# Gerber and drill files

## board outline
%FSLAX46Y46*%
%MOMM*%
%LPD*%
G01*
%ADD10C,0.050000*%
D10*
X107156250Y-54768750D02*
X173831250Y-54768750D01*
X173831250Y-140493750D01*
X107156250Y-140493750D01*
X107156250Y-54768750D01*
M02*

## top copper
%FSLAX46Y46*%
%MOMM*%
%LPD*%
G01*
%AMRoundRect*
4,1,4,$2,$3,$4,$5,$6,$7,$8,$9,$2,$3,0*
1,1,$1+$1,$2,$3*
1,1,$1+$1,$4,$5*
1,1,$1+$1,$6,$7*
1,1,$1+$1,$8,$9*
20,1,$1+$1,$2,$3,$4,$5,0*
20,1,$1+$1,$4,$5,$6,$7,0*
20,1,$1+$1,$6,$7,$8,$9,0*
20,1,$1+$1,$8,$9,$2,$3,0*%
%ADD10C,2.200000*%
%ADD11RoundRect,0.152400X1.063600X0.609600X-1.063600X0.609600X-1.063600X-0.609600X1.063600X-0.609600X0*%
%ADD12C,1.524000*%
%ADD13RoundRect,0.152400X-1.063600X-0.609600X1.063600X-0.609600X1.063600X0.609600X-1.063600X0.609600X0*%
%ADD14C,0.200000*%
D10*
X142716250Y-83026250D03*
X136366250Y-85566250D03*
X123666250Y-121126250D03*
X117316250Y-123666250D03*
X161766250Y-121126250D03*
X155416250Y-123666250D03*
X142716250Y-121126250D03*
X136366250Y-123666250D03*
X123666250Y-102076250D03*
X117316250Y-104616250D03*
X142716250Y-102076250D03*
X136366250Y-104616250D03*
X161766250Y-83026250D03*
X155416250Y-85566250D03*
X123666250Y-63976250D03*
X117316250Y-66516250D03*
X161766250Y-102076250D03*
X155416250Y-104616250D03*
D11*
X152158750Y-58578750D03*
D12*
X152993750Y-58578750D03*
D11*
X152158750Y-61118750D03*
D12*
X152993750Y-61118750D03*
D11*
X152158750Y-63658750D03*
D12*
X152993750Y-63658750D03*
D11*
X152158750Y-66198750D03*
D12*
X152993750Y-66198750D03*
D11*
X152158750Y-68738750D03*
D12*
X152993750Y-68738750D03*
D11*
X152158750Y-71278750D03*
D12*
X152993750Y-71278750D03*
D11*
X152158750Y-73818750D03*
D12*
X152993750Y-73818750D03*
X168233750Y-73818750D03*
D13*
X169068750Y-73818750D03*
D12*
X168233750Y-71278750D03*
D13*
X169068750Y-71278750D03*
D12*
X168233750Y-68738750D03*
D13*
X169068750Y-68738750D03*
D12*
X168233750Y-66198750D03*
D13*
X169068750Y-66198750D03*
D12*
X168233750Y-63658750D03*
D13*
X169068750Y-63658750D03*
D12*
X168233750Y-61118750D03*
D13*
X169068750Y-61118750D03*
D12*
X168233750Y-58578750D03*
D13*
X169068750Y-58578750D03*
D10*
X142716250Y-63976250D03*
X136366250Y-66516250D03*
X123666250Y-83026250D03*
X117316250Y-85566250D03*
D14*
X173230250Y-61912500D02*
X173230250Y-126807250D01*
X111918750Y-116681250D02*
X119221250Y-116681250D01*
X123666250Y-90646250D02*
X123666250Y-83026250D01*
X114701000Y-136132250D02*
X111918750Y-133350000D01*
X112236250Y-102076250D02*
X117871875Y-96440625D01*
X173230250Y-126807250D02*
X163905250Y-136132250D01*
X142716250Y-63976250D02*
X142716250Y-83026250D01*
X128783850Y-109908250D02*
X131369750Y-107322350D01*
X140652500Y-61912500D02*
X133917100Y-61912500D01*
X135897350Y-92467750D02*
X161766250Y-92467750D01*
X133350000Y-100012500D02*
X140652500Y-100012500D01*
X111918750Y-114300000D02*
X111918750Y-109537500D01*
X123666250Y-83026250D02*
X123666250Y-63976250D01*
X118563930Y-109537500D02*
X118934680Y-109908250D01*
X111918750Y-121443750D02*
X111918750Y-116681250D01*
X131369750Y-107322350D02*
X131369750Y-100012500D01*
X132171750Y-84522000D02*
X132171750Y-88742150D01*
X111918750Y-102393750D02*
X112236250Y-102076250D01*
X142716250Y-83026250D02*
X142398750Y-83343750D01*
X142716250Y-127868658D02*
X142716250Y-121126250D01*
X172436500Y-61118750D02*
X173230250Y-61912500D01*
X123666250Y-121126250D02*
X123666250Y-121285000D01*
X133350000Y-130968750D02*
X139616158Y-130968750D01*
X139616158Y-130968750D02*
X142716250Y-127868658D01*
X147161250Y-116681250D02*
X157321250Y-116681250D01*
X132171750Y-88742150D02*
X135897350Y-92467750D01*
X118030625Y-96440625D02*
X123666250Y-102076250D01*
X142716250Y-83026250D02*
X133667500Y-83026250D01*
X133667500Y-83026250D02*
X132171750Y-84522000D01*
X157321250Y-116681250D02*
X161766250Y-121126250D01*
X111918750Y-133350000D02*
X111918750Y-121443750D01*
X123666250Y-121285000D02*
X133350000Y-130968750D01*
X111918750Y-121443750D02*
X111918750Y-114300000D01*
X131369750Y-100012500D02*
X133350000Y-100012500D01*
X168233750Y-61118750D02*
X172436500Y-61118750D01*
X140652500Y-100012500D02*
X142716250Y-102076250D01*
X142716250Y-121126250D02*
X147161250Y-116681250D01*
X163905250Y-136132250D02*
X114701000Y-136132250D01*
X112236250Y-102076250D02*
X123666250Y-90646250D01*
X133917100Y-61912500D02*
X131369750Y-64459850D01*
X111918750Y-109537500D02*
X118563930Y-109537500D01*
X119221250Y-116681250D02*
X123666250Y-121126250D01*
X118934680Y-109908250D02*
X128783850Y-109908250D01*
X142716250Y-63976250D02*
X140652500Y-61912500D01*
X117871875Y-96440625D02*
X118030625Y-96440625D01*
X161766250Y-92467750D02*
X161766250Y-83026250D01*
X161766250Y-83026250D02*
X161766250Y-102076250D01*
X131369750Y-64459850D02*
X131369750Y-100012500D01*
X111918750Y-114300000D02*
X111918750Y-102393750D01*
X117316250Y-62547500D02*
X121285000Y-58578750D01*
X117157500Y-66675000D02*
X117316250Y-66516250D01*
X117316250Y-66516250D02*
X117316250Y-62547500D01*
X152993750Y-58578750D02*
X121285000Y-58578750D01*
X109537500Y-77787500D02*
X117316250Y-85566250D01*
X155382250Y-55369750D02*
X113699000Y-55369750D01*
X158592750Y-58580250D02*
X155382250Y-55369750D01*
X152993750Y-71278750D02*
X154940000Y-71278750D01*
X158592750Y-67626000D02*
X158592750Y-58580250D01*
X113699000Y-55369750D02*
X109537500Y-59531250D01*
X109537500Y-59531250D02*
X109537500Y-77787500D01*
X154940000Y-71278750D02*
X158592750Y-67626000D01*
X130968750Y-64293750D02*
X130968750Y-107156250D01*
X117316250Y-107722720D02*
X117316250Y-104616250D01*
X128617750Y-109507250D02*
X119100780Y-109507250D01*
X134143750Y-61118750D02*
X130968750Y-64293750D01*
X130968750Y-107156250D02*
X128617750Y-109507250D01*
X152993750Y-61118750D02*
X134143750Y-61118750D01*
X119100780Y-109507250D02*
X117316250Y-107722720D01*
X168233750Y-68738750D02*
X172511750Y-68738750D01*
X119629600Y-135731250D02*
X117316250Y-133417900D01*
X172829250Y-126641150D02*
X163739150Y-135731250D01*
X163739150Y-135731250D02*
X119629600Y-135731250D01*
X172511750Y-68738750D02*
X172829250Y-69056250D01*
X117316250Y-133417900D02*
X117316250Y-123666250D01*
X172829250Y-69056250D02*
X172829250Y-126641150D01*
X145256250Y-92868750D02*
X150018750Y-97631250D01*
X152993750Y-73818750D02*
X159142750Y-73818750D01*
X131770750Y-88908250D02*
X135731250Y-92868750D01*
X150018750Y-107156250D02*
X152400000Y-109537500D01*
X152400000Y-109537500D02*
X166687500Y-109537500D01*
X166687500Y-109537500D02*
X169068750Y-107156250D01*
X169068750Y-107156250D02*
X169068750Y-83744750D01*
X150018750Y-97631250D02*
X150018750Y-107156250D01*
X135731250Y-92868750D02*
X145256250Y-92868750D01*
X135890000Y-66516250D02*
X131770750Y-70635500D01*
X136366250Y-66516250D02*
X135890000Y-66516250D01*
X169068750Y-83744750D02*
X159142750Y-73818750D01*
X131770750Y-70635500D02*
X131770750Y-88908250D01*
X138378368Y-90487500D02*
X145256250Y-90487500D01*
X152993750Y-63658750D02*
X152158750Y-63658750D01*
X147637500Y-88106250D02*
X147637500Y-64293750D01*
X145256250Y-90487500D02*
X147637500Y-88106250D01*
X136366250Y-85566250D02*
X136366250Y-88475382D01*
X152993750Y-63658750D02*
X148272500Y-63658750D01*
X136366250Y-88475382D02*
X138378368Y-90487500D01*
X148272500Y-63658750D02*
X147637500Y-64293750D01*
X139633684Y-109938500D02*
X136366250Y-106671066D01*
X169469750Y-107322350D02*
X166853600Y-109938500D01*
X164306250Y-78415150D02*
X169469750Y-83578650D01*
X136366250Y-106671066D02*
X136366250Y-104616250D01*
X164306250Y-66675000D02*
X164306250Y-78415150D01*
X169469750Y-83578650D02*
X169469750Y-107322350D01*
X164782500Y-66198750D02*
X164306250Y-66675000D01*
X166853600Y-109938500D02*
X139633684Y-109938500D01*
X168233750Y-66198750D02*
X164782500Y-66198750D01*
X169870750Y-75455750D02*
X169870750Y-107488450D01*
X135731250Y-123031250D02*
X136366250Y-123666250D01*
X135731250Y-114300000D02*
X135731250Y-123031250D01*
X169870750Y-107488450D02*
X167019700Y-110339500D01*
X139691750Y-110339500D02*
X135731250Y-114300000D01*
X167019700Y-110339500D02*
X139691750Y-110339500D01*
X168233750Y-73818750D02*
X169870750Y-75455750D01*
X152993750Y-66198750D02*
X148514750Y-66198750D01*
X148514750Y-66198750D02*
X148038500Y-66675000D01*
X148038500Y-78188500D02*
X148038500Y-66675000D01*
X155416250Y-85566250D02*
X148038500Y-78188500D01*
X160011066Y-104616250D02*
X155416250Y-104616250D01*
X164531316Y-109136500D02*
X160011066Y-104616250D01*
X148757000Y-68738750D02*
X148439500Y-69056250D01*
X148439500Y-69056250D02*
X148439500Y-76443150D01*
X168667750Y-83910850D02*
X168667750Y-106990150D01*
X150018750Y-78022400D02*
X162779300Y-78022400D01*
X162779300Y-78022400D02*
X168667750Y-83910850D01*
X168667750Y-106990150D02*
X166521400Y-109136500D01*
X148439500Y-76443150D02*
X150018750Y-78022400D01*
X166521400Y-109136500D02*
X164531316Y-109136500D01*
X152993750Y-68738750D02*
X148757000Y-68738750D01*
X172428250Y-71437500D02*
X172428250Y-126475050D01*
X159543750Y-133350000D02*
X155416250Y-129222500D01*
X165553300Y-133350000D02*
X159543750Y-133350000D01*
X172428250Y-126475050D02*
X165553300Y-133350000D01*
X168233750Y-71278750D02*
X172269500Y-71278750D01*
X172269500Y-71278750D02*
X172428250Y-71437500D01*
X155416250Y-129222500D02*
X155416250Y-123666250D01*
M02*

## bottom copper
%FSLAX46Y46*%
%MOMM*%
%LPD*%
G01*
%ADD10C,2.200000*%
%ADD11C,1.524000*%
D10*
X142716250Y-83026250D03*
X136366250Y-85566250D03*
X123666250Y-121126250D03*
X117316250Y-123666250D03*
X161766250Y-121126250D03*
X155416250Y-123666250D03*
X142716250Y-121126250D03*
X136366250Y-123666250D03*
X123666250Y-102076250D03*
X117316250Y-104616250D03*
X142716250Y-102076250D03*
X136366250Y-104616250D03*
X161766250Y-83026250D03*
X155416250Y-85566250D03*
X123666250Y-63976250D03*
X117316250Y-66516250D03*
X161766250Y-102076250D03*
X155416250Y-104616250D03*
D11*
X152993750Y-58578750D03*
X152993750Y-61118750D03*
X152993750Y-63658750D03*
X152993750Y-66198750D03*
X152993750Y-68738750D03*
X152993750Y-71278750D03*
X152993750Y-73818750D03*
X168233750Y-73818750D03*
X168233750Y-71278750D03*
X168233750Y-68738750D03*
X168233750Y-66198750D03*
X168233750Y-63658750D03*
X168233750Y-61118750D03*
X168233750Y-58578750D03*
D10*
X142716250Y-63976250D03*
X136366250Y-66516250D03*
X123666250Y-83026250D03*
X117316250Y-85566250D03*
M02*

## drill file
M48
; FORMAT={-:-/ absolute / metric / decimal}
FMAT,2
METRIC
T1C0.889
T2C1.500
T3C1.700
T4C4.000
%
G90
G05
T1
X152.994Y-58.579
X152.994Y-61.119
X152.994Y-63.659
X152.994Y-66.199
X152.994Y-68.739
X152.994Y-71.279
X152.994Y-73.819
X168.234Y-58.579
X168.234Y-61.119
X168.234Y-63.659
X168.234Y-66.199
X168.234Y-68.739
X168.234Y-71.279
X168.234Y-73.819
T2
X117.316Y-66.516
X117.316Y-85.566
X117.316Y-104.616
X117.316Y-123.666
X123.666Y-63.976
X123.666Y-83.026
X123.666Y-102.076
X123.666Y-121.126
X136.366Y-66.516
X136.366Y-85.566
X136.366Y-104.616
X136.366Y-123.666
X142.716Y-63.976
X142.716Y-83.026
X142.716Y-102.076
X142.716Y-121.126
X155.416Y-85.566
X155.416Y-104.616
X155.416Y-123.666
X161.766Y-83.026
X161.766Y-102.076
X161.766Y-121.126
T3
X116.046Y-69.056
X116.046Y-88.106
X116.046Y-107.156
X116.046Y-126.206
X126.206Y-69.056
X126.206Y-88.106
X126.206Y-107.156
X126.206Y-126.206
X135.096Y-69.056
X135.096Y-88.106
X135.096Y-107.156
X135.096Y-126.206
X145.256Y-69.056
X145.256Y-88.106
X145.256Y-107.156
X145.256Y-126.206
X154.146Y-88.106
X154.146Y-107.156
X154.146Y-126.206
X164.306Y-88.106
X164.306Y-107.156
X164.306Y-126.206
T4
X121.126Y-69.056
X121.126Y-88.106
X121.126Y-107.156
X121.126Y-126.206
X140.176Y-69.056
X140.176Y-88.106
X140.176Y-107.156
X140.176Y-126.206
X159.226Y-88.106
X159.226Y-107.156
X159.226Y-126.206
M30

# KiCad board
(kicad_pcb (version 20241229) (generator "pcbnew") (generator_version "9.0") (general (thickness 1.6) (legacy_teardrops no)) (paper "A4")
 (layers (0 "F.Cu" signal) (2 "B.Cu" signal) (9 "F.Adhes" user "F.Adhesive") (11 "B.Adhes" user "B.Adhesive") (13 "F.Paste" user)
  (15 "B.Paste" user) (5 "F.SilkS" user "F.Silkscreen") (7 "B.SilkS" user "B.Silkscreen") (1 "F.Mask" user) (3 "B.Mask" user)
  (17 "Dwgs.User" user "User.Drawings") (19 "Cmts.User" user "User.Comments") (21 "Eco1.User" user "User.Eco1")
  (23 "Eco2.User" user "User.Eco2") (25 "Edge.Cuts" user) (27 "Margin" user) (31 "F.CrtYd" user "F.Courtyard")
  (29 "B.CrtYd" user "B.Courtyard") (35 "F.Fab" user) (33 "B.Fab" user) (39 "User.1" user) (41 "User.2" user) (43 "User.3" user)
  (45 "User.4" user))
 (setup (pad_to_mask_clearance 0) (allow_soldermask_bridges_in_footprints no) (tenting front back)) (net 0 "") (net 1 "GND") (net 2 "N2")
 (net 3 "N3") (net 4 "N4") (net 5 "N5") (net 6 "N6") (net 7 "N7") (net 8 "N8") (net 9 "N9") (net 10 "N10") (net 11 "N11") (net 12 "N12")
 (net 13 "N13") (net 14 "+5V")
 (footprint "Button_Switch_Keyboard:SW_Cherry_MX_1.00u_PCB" (layer "F.Cu") (at 142.71625 83.02625)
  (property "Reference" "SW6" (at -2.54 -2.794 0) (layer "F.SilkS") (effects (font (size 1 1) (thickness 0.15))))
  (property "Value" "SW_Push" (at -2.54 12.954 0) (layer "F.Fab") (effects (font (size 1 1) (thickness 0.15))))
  (pad "" np_thru_hole circle (at -7.62 5.08) (size 1.7 1.7) (drill 1.7) (layers "*.Cu" "*.Mask"))
  (pad "" np_thru_hole circle (at -2.54 5.08) (size 4 4) (drill 4) (layers "*.Cu" "*.Mask"))
  (pad "" np_thru_hole circle (at 2.54 5.08) (size 1.7 1.7) (drill 1.7) (layers "*.Cu" "*.Mask"))
  (pad "1" thru_hole circle (at 0 0) (size 2.2 2.2) (drill 1.5) (layers "*.Cu" "*.Mask") (remove_unused_layers no) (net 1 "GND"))
  (pad "2" thru_hole circle (at -6.35 2.54) (size 2.2 2.2) (drill 1.5) (layers "*.Cu" "*.Mask") (remove_unused_layers no) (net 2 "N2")))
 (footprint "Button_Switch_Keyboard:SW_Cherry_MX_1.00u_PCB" (layer "F.Cu") (at 123.66625 121.12625)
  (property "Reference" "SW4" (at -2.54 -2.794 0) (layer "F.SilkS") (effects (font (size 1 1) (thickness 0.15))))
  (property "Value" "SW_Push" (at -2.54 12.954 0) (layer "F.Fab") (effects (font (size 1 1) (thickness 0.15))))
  (pad "" np_thru_hole circle (at -7.62 5.08) (size 1.7 1.7) (drill 1.7) (layers "*.Cu" "*.Mask"))
  (pad "" np_thru_hole circle (at -2.54 5.08) (size 4 4) (drill 4) (layers "*.Cu" "*.Mask"))
  (pad "" np_thru_hole circle (at 2.54 5.08) (size 1.7 1.7) (drill 1.7) (layers "*.Cu" "*.Mask"))
  (pad "1" thru_hole circle (at 0 0) (size 2.2 2.2) (drill 1.5) (layers "*.Cu" "*.Mask") (remove_unused_layers no) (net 1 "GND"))
  (pad "2" thru_hole circle (at -6.35 2.54) (size 2.2 2.2) (drill 1.5) (layers "*.Cu" "*.Mask") (remove_unused_layers no) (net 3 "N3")))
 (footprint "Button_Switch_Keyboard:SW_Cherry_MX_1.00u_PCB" (layer "F.Cu") (at 161.76625 121.12625)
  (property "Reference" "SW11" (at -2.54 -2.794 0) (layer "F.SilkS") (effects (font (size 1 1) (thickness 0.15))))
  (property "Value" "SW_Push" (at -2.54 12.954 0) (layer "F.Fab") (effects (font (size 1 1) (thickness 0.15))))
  (pad "" np_thru_hole circle (at -7.62 5.08) (size 1.7 1.7) (drill 1.7) (layers "*.Cu" "*.Mask"))
  (pad "" np_thru_hole circle (at -2.54 5.08) (size 4 4) (drill 4) (layers "*.Cu" "*.Mask"))
  (pad "" np_thru_hole circle (at 2.54 5.08) (size 1.7 1.7) (drill 1.7) (layers "*.Cu" "*.Mask"))
  (pad "1" thru_hole circle (at 0 0) (size 2.2 2.2) (drill 1.5) (layers "*.Cu" "*.Mask") (remove_unused_layers no) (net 1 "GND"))
  (pad "2" thru_hole circle (at -6.35 2.54) (size 2.2 2.2) (drill 1.5) (layers "*.Cu" "*.Mask") (remove_unused_layers no) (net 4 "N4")))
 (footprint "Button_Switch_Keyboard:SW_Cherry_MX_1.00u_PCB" (layer "F.Cu") (at 142.71625 121.12625)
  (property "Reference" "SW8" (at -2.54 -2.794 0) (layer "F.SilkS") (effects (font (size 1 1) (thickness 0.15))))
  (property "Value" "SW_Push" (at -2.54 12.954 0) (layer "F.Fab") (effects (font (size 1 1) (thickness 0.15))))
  (pad "" np_thru_hole circle (at -7.62 5.08) (size 1.7 1.7) (drill 1.7) (layers "*.Cu" "*.Mask"))
  (pad "" np_thru_hole circle (at -2.54 5.08) (size 4 4) (drill 4) (layers "*.Cu" "*.Mask"))
  (pad "" np_thru_hole circle (at 2.54 5.08) (size 1.7 1.7) (drill 1.7) (layers "*.Cu" "*.Mask"))
  (pad "1" thru_hole circle (at 0 0) (size 2.2 2.2) (drill 1.5) (layers "*.Cu" "*.Mask") (remove_unused_layers no) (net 1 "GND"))
  (pad "2" thru_hole circle (at -6.35 2.54) (size 2.2 2.2) (drill 1.5) (layers "*.Cu" "*.Mask") (remove_unused_layers no) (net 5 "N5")))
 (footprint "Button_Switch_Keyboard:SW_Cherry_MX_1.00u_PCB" (layer "F.Cu") (at 123.66625 102.07625)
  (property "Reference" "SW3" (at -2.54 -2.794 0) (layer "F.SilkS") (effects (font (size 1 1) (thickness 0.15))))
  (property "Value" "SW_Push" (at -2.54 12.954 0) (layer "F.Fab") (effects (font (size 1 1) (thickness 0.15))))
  (pad "" np_thru_hole circle (at -7.62 5.08) (size 1.7 1.7) (drill 1.7) (layers "*.Cu" "*.Mask"))
  (pad "" np_thru_hole circle (at -2.54 5.08) (size 4 4) (drill 4) (layers "*.Cu" "*.Mask"))
  (pad "" np_thru_hole circle (at 2.54 5.08) (size 1.7 1.7) (drill 1.7) (layers "*.Cu" "*.Mask"))
  (pad "1" thru_hole circle (at 0 0) (size 2.2 2.2) (drill 1.5) (layers "*.Cu" "*.Mask") (remove_unused_layers no) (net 1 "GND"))
  (pad "2" thru_hole circle (at -6.35 2.54) (size 2.2 2.2) (drill 1.5) (layers "*.Cu" "*.Mask") (remove_unused_layers no) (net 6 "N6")))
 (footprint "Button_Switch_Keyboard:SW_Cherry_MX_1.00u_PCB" (layer "F.Cu") (at 142.71625 102.07625)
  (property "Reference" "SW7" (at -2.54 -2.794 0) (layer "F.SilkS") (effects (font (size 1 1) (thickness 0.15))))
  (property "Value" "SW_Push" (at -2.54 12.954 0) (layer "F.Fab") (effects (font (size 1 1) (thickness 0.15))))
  (pad "" np_thru_hole circle (at -7.62 5.08) (size 1.7 1.7) (drill 1.7) (layers "*.Cu" "*.Mask"))
  (pad "" np_thru_hole circle (at -2.54 5.08) (size 4 4) (drill 4) (layers "*.Cu" "*.Mask"))
  (pad "" np_thru_hole circle (at 2.54 5.08) (size 1.7 1.7) (drill 1.7) (layers "*.Cu" "*.Mask"))
  (pad "1" thru_hole circle (at 0 0) (size 2.2 2.2) (drill 1.5) (layers "*.Cu" "*.Mask") (remove_unused_layers no) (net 1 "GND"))
  (pad "2" thru_hole circle (at -6.35 2.54) (size 2.2 2.2) (drill 1.5) (layers "*.Cu" "*.Mask") (remove_unused_layers no) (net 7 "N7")))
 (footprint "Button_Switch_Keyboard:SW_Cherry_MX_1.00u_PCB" (layer "F.Cu") (at 161.76625 83.02625)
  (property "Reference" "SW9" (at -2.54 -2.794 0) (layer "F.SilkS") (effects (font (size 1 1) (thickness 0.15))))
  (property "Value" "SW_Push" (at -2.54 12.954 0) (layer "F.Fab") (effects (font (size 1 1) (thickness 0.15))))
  (pad "" np_thru_hole circle (at -7.62 5.08) (size 1.7 1.7) (drill 1.7) (layers "*.Cu" "*.Mask"))
  (pad "" np_thru_hole circle (at -2.54 5.08) (size 4 4) (drill 4) (layers "*.Cu" "*.Mask"))
  (pad "" np_thru_hole circle (at 2.54 5.08) (size 1.7 1.7) (drill 1.7) (layers "*.Cu" "*.Mask"))
  (pad "1" thru_hole circle (at 0 0) (size 2.2 2.2) (drill 1.5) (layers "*.Cu" "*.Mask") (remove_unused_layers no) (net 1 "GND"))
  (pad "2" thru_hole circle (at -6.35 2.54) (size 2.2 2.2) (drill 1.5) (layers "*.Cu" "*.Mask") (remove_unused_layers no) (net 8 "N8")))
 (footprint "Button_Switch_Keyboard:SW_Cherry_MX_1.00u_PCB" (layer "F.Cu") (at 123.66625 63.97625)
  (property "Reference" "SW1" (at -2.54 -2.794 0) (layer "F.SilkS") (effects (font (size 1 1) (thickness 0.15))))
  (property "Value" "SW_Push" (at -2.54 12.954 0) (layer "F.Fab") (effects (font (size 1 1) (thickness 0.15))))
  (pad "" np_thru_hole circle (at -7.62 5.08) (size 1.7 1.7) (drill 1.7) (layers "*.Cu" "*.Mask"))
  (pad "" np_thru_hole circle (at -2.54 5.08) (size 4 4) (drill 4) (layers "*.Cu" "*.Mask"))
  (pad "" np_thru_hole circle (at 2.54 5.08) (size 1.7 1.7) (drill 1.7) (layers "*.Cu" "*.Mask"))
  (pad "1" thru_hole circle (at 0 0) (size 2.2 2.2) (drill 1.5) (layers "*.Cu" "*.Mask") (remove_unused_layers no) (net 1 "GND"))
  (pad "2" thru_hole circle (at -6.35 2.54) (size 2.2 2.2) (drill 1.5) (layers "*.Cu" "*.Mask") (remove_unused_layers no) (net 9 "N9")))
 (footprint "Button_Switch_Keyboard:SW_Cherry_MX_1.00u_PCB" (layer "F.Cu") (at 161.76625 102.07625)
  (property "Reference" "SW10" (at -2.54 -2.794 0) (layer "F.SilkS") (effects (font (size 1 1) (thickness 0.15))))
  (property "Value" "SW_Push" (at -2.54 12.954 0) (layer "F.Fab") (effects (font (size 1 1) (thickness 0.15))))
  (pad "" np_thru_hole circle (at -7.62 5.08) (size 1.7 1.7) (drill 1.7) (layers "*.Cu" "*.Mask"))
  (pad "" np_thru_hole circle (at -2.54 5.08) (size 4 4) (drill 4) (layers "*.Cu" "*.Mask"))
  (pad "" np_thru_hole circle (at 2.54 5.08) (size 1.7 1.7) (drill 1.7) (layers "*.Cu" "*.Mask"))
  (pad "1" thru_hole circle (at 0 0) (size 2.2 2.2) (drill 1.5) (layers "*.Cu" "*.Mask") (remove_unused_layers no) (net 1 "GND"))
  (pad "2" thru_hole circle (at -6.35 2.54) (size 2.2 2.2) (drill 1.5) (layers "*.Cu" "*.Mask") (remove_unused_layers no) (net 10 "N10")))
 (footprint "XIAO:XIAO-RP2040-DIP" (layer "F.Cu") (at 160.61375 66.19875)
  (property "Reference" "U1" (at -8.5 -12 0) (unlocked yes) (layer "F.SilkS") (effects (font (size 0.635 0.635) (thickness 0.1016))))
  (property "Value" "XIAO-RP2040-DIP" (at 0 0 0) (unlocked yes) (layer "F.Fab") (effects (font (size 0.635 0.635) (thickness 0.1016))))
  (pad "1" smd roundrect (at -8.455 -7.62 180) (size 2.432 1.524) (layers "F.Cu" "F.Mask") (roundrect_rratio 0.1) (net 9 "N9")
   (thermal_bridge_angle 45))
  (pad "1" thru_hole circle (at -7.62 -7.62 180) (size 1.524 1.524) (drill 0.889) (layers "*.Cu" "*.Mask") (remove_unused_layers no)
   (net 9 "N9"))
  (pad "2" smd roundrect (at -8.455 -5.08 180) (size 2.432 1.524) (layers "F.Cu" "F.Mask") (roundrect_rratio 0.1) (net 6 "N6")
   (thermal_bridge_angle 45))
  (pad "2" thru_hole circle (at -7.62 -5.08 180) (size 1.524 1.524) (drill 0.889) (layers "*.Cu" "*.Mask") (remove_unused_layers no)
   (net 6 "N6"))
  (pad "3" smd roundrect (at -8.455 -2.54 180) (size 2.432 1.524) (layers "F.Cu" "F.Mask") (roundrect_rratio 0.1) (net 2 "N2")
   (thermal_bridge_angle 45))
  (pad "3" thru_hole circle (at -7.62 -2.54 180) (size 1.524 1.524) (drill 0.889) (layers "*.Cu" "*.Mask") (remove_unused_layers no)
   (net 2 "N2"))
  (pad "4" smd roundrect (at -8.455 0 180) (size 2.432 1.524) (layers "F.Cu" "F.Mask") (roundrect_rratio 0.1) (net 8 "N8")
   (thermal_bridge_angle 45))
  (pad "4" thru_hole circle (at -7.62 0 180) (size 1.524 1.524) (drill 0.889) (layers "*.Cu" "*.Mask") (remove_unused_layers no)
   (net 8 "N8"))
  (pad "5" smd roundrect (at -8.455 2.54 180) (size 2.432 1.524) (layers "F.Cu" "F.Mask") (roundrect_rratio 0.1) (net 10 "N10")
   (thermal_bridge_angle 45))
  (pad "5" thru_hole circle (at -7.62 2.54 180) (size 1.524 1.524) (drill 0.889) (layers "*.Cu" "*.Mask") (remove_unused_layers no)
   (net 10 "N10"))
  (pad "6" smd roundrect (at -8.455 5.08 180) (size 2.432 1.524) (layers "F.Cu" "F.Mask") (roundrect_rratio 0.1) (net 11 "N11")
   (thermal_bridge_angle 45))
  (pad "6" thru_hole circle (at -7.62 5.08 180) (size 1.524 1.524) (drill 0.889) (layers "*.Cu" "*.Mask") (remove_unused_layers no)
   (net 11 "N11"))
  (pad "7" smd roundrect (at -8.455 7.62 180) (size 2.432 1.524) (layers "F.Cu" "F.Mask") (roundrect_rratio 0.1) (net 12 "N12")
   (thermal_bridge_angle 45))
  (pad "7" thru_hole circle (at -7.62 7.62 180) (size 1.524 1.524) (drill 0.889) (layers "*.Cu" "*.Mask") (remove_unused_layers no)
   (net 12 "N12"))
  (pad "8" thru_hole circle (at 7.62 7.62) (size 1.524 1.524) (drill 0.889) (layers "*.Cu" "*.Mask") (remove_unused_layers no) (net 5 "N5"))
  (pad "8" smd roundrect (at 8.455 7.62) (size 2.432 1.524) (layers "F.Cu" "F.Mask") (roundrect_rratio 0.1) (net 5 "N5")
   (thermal_bridge_angle 45))
  (pad "9" thru_hole circle (at 7.62 5.08) (size 1.524 1.524) (drill 0.889) (layers "*.Cu" "*.Mask") (remove_unused_layers no) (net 4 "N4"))
  (pad "9" smd roundrect (at 8.455 5.08) (size 2.432 1.524) (layers "F.Cu" "F.Mask") (roundrect_rratio 0.1) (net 4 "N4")
   (thermal_bridge_angle 45))
  (pad "10" thru_hole circle (at 7.62 2.54) (size 1.524 1.524) (drill 0.889) (layers "*.Cu" "*.Mask") (remove_unused_layers no) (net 3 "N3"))
  (pad "10" smd roundrect (at 8.455 2.54) (size 2.432 1.524) (layers "F.Cu" "F.Mask") (roundrect_rratio 0.1) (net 3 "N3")
   (thermal_bridge_angle 45))
  (pad "11" thru_hole circle (at 7.62 0) (size 1.524 1.524) (drill 0.889) (layers "*.Cu" "*.Mask") (remove_unused_layers no) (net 7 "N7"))
  (pad "11" smd roundrect (at 8.455 0) (size 2.432 1.524) (layers "F.Cu" "F.Mask") (roundrect_rratio 0.1) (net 7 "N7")
   (thermal_bridge_angle 45))
  (pad "12" thru_hole circle (at 7.62 -2.54) (size 1.524 1.524) (drill 0.889) (layers "*.Cu" "*.Mask") (remove_unused_layers no)
   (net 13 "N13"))
  (pad "12" smd roundrect (at 8.455 -2.54) (size 2.432 1.524) (layers "F.Cu" "F.Mask") (roundrect_rratio 0.1) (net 13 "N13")
   (thermal_bridge_angle 45))
  (pad "13" thru_hole circle (at 7.62 -5.08) (size 1.524 1.524) (drill 0.889) (layers "*.Cu" "*.Mask") (remove_unused_layers no)
   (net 1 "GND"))
  (pad "13" smd roundrect (at 8.455 -5.08) (size 2.432 1.524) (layers "F.Cu" "F.Mask") (roundrect_rratio 0.1) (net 1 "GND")
   (thermal_bridge_angle 45))
  (pad "14" thru_hole circle (at 7.62 -7.62) (size 1.524 1.524) (drill 0.889) (layers "*.Cu" "*.Mask") (remove_unused_layers no)
   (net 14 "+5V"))
  (pad "14" smd roundrect (at 8.455 -7.62) (size 2.432 1.524) (layers "F.Cu" "F.Mask") (roundrect_rratio 0.1) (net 14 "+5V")
   (thermal_bridge_angle 45)))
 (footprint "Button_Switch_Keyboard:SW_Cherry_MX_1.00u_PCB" (layer "F.Cu") (at 142.71625 63.97625)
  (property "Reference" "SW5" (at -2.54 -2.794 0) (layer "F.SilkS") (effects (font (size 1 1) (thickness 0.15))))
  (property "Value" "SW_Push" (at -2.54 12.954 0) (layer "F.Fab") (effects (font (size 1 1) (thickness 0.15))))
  (pad "" np_thru_hole circle (at -7.62 5.08) (size 1.7 1.7) (drill 1.7) (layers "*.Cu" "*.Mask"))
  (pad "" np_thru_hole circle (at -2.54 5.08) (size 4 4) (drill 4) (layers "*.Cu" "*.Mask"))
  (pad "" np_thru_hole circle (at 2.54 5.08) (size 1.7 1.7) (drill 1.7) (layers "*.Cu" "*.Mask"))
  (pad "1" thru_hole circle (at 0 0) (size 2.2 2.2) (drill 1.5) (layers "*.Cu" "*.Mask") (remove_unused_layers no) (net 1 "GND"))
  (pad "2" thru_hole circle (at -6.35 2.54) (size 2.2 2.2) (drill 1.5) (layers "*.Cu" "*.Mask") (remove_unused_layers no) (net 12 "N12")))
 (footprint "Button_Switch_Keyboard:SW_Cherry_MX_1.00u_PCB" (layer "F.Cu") (at 123.66625 83.02625)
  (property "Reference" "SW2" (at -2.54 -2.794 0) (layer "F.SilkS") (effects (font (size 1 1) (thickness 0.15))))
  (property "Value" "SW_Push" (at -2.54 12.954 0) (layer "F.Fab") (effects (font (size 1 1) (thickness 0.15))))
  (pad "" np_thru_hole circle (at -7.62 5.08) (size 1.7 1.7) (drill 1.7) (layers "*.Cu" "*.Mask"))
  (pad "" np_thru_hole circle (at -2.54 5.08) (size 4 4) (drill 4) (layers "*.Cu" "*.Mask"))
  (pad "" np_thru_hole circle (at 2.54 5.08) (size 1.7 1.7) (drill 1.7) (layers "*.Cu" "*.Mask"))
  (pad "1" thru_hole circle (at 0 0) (size 2.2 2.2) (drill 1.5) (layers "*.Cu" "*.Mask") (remove_unused_layers no) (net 1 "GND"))
  (pad "2" thru_hole circle (at -6.35 2.54) (size 2.2 2.2) (drill 1.5) (layers "*.Cu" "*.Mask") (remove_unused_layers no) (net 11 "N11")))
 (gr_rect (start 107.15625 54.76875) (end 173.83125 140.49375) (stroke (width 0.05) (type default)) (fill no) (layer "Edge.Cuts"))
 (segment (start 173.23025 61.9125) (end 173.23025 126.80725) (width 0.2) (layer "F.Cu") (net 1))
 (segment (start 111.91875 116.68125) (end 119.22125 116.68125) (width 0.2) (layer "F.Cu") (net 1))
 (segment (start 123.66625 90.64625) (end 123.66625 83.02625) (width 0.2) (layer "F.Cu") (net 1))
 (segment (start 114.701 136.13225) (end 111.91875 133.35) (width 0.2) (layer "F.Cu") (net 1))
 (segment (start 112.23625 102.07625) (end 117.871875 96.440625) (width 0.2) (layer "F.Cu") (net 1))
 (segment (start 173.23025 126.80725) (end 163.90525 136.13225) (width 0.2) (layer "F.Cu") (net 1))
 (segment (start 142.71625 63.97625) (end 142.71625 83.02625) (width 0.2) (layer "F.Cu") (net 1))
 (segment (start 128.78385 109.90825) (end 131.36975 107.32235) (width 0.2) (layer "F.Cu") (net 1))
 (segment (start 140.6525 61.9125) (end 133.9171 61.9125) (width 0.2) (layer "F.Cu") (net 1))
 (segment (start 135.89735 92.46775) (end 161.76625 92.46775) (width 0.2) (layer "F.Cu") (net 1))
 (segment (start 133.35 100.0125) (end 140.6525 100.0125) (width 0.2) (layer "F.Cu") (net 1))
 (segment (start 111.91875 114.3) (end 111.91875 109.5375) (width 0.2) (layer "F.Cu") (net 1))
 (segment (start 123.66625 83.02625) (end 123.66625 63.97625) (width 0.2) (layer "F.Cu") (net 1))
 (segment (start 118.56393 109.5375) (end 118.93468 109.90825) (width 0.2) (layer "F.Cu") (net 1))
 (segment (start 111.91875 121.44375) (end 111.91875 116.68125) (width 0.2) (layer "F.Cu") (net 1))
 (segment (start 131.36975 107.32235) (end 131.36975 100.0125) (width 0.2) (layer "F.Cu") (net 1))
 (segment (start 132.17175 84.522) (end 132.17175 88.74215) (width 0.2) (layer "F.Cu") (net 1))
 (segment (start 111.91875 102.39375) (end 112.23625 102.07625) (width 0.2) (layer "F.Cu") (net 1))
 (segment (start 142.71625 83.02625) (end 142.39875 83.34375) (width 0.2) (layer "F.Cu") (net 1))
 (segment (start 142.71625 127.868658) (end 142.71625 121.12625) (width 0.2) (layer "F.Cu") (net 1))
 (segment (start 172.4365 61.11875) (end 173.23025 61.9125) (width 0.2) (layer "F.Cu") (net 1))
 (segment (start 123.66625 121.12625) (end 123.66625 121.285) (width 0.2) (layer "F.Cu") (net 1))
 (segment (start 133.35 130.96875) (end 139.616158 130.96875) (width 0.2) (layer "F.Cu") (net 1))
 (segment (start 139.616158 130.96875) (end 142.71625 127.868658) (width 0.2) (layer "F.Cu") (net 1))
 (segment (start 147.16125 116.68125) (end 157.32125 116.68125) (width 0.2) (layer "F.Cu") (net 1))
 (segment (start 132.17175 88.74215) (end 135.89735 92.46775) (width 0.2) (layer "F.Cu") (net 1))
 (segment (start 118.030625 96.440625) (end 123.66625 102.07625) (width 0.2) (layer "F.Cu") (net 1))
 (segment (start 142.71625 83.02625) (end 133.6675 83.02625) (width 0.2) (layer "F.Cu") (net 1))
 (segment (start 133.6675 83.02625) (end 132.17175 84.522) (width 0.2) (layer "F.Cu") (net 1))
 (segment (start 157.32125 116.68125) (end 161.76625 121.12625) (width 0.2) (layer "F.Cu") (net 1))
 (segment (start 111.91875 133.35) (end 111.91875 121.44375) (width 0.2) (layer "F.Cu") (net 1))
 (segment (start 123.66625 121.285) (end 133.35 130.96875) (width 0.2) (layer "F.Cu") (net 1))
 (segment (start 111.91875 121.44375) (end 111.91875 114.3) (width 0.2) (layer "F.Cu") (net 1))
 (segment (start 131.36975 100.0125) (end 133.35 100.0125) (width 0.2) (layer "F.Cu") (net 1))
 (segment (start 168.23375 61.11875) (end 172.4365 61.11875) (width 0.2) (layer "F.Cu") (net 1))
 (segment (start 140.6525 100.0125) (end 142.71625 102.07625) (width 0.2) (layer "F.Cu") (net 1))
 (segment (start 142.71625 121.12625) (end 147.16125 116.68125) (width 0.2) (layer "F.Cu") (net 1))
 (segment (start 163.90525 136.13225) (end 114.701 136.13225) (width 0.2) (layer "F.Cu") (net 1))
 (segment (start 112.23625 102.07625) (end 123.66625 90.64625) (width 0.2) (layer "F.Cu") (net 1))
 (segment (start 133.9171 61.9125) (end 131.36975 64.45985) (width 0.2) (layer "F.Cu") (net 1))
 (segment (start 111.91875 109.5375) (end 118.56393 109.5375) (width 0.2) (layer "F.Cu") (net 1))
 (segment (start 119.22125 116.68125) (end 123.66625 121.12625) (width 0.2) (layer "F.Cu") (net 1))
 (segment (start 118.93468 109.90825) (end 128.78385 109.90825) (width 0.2) (layer "F.Cu") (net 1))
 (segment (start 142.71625 63.97625) (end 140.6525 61.9125) (width 0.2) (layer "F.Cu") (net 1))
 (segment (start 117.871875 96.440625) (end 118.030625 96.440625) (width 0.2) (layer "F.Cu") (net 1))
 (segment (start 161.76625 92.46775) (end 161.76625 83.02625) (width 0.2) (layer "F.Cu") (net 1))
 (segment (start 161.76625 83.02625) (end 161.76625 102.07625) (width 0.2) (layer "F.Cu") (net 1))
 (segment (start 131.36975 64.45985) (end 131.36975 100.0125) (width 0.2) (layer "F.Cu") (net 1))
 (segment (start 111.91875 114.3) (end 111.91875 102.39375) (width 0.2) (layer "F.Cu") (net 1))
 (segment (start 117.31625 62.5475) (end 121.285 58.57875) (width 0.2) (layer "F.Cu") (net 9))
 (segment (start 117.1575 66.675) (end 117.31625 66.51625) (width 0.2) (layer "F.Cu") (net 9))
 (segment (start 117.31625 66.51625) (end 117.31625 62.5475) (width 0.2) (layer "F.Cu") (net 9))
 (segment (start 152.99375 58.57875) (end 121.285 58.57875) (width 0.2) (layer "F.Cu") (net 9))
 (segment (start 109.5375 77.7875) (end 117.31625 85.56625) (width 0.2) (layer "F.Cu") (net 11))
 (segment (start 155.38225 55.36975) (end 113.699 55.36975) (width 0.2) (layer "F.Cu") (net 11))
 (segment (start 158.59275 58.58025) (end 155.38225 55.36975) (width 0.2) (layer "F.Cu") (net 11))
 (segment (start 152.99375 71.27875) (end 154.94 71.27875) (width 0.2) (layer "F.Cu") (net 11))
 (segment (start 158.59275 67.626) (end 158.59275 58.58025) (width 0.2) (layer "F.Cu") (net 11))
 (segment (start 113.699 55.36975) (end 109.5375 59.53125) (width 0.2) (layer "F.Cu") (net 11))
 (segment (start 109.5375 59.53125) (end 109.5375 77.7875) (width 0.2) (layer "F.Cu") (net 11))
 (segment (start 154.94 71.27875) (end 158.59275 67.626) (width 0.2) (layer "F.Cu") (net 11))
 (segment (start 130.96875 64.29375) (end 130.96875 107.15625) (width 0.2) (layer "F.Cu") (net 6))
 (segment (start 117.31625 107.72272) (end 117.31625 104.61625) (width 0.2) (layer "F.Cu") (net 6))
 (segment (start 128.61775 109.50725) (end 119.10078 109.50725) (width 0.2) (layer "F.Cu") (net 6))
 (segment (start 134.14375 61.11875) (end 130.96875 64.29375) (width 0.2) (layer "F.Cu") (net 6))
 (segment (start 130.96875 107.15625) (end 128.61775 109.50725) (width 0.2) (layer "F.Cu") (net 6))
 (segment (start 152.99375 61.11875) (end 134.14375 61.11875) (width 0.2) (layer "F.Cu") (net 6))
 (segment (start 119.10078 109.50725) (end 117.31625 107.72272) (width 0.2) (layer "F.Cu") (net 6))
 (segment (start 168.23375 68.73875) (end 172.51175 68.73875) (width 0.2) (layer "F.Cu") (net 3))
 (segment (start 119.6296 135.73125) (end 117.31625 133.4179) (width 0.2) (layer "F.Cu") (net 3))
 (segment (start 172.82925 126.64115) (end 163.73915 135.73125) (width 0.2) (layer "F.Cu") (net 3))
 (segment (start 163.73915 135.73125) (end 119.6296 135.73125) (width 0.2) (layer "F.Cu") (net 3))
 (segment (start 172.51175 68.73875) (end 172.82925 69.05625) (width 0.2) (layer "F.Cu") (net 3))
 (segment (start 117.31625 133.4179) (end 117.31625 123.66625) (width 0.2) (layer "F.Cu") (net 3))
 (segment (start 172.82925 69.05625) (end 172.82925 126.64115) (width 0.2) (layer "F.Cu") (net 3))
 (segment (start 145.25625 92.86875) (end 150.01875 97.63125) (width 0.2) (layer "F.Cu") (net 12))
 (segment (start 152.99375 73.81875) (end 159.14275 73.81875) (width 0.2) (layer "F.Cu") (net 12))
 (segment (start 131.77075 88.90825) (end 135.73125 92.86875) (width 0.2) (layer "F.Cu") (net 12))
 (segment (start 150.01875 107.15625) (end 152.4 109.5375) (width 0.2) (layer "F.Cu") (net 12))
 (segment (start 152.4 109.5375) (end 166.6875 109.5375) (width 0.2) (layer "F.Cu") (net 12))
 (segment (start 166.6875 109.5375) (end 169.06875 107.15625) (width 0.2) (layer "F.Cu") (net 12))
 (segment (start 169.06875 107.15625) (end 169.06875 83.74475) (width 0.2) (layer "F.Cu") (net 12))
 (segment (start 150.01875 97.63125) (end 150.01875 107.15625) (width 0.2) (layer "F.Cu") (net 12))
 (segment (start 135.73125 92.86875) (end 145.25625 92.86875) (width 0.2) (layer "F.Cu") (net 12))
 (segment (start 135.89 66.51625) (end 131.77075 70.6355) (width 0.2) (layer "F.Cu") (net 12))
 (segment (start 136.36625 66.51625) (end 135.89 66.51625) (width 0.2) (layer "F.Cu") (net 12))
 (segment (start 169.06875 83.74475) (end 159.14275 73.81875) (width 0.2) (layer "F.Cu") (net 12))
 (segment (start 131.77075 70.6355) (end 131.77075 88.90825) (width 0.2) (layer "F.Cu") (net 12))
 (segment (start 138.378368 90.4875) (end 145.25625 90.4875) (width 0.2) (layer "F.Cu") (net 2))
 (segment (start 152.99375 63.65875) (end 152.15875 63.65875) (width 0.2) (layer "F.Cu") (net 2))
 (segment (start 147.6375 88.10625) (end 147.6375 64.29375) (width 0.2) (layer "F.Cu") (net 2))
 (segment (start 145.25625 90.4875) (end 147.6375 88.10625) (width 0.2) (layer "F.Cu") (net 2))
 (segment (start 136.36625 85.56625) (end 136.36625 88.475382) (width 0.2) (layer "F.Cu") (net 2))
 (segment (start 152.99375 63.65875) (end 148.2725 63.65875) (width 0.2) (layer "F.Cu") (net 2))
 (segment (start 136.36625 88.475382) (end 138.378368 90.4875) (width 0.2) (layer "F.Cu") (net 2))
 (segment (start 148.2725 63.65875) (end 147.6375 64.29375) (width 0.2) (layer "F.Cu") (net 2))
 (segment (start 139.633684 109.9385) (end 136.36625 106.671066) (width 0.2) (layer "F.Cu") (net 7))
 (segment (start 169.46975 107.32235) (end 166.8536 109.9385) (width 0.2) (layer "F.Cu") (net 7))
 (segment (start 164.30625 78.41515) (end 169.46975 83.57865) (width 0.2) (layer "F.Cu") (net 7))
 (segment (start 136.36625 106.671066) (end 136.36625 104.61625) (width 0.2) (layer "F.Cu") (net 7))
 (segment (start 164.30625 66.675) (end 164.30625 78.41515) (width 0.2) (layer "F.Cu") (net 7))
 (segment (start 169.46975 83.57865) (end 169.46975 107.32235) (width 0.2) (layer "F.Cu") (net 7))
 (segment (start 164.7825 66.19875) (end 164.30625 66.675) (width 0.2) (layer "F.Cu") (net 7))
 (segment (start 166.8536 109.9385) (end 139.633684 109.9385) (width 0.2) (layer "F.Cu") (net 7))
 (segment (start 168.23375 66.19875) (end 164.7825 66.19875) (width 0.2) (layer "F.Cu") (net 7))
 (segment (start 169.87075 75.45575) (end 169.87075 107.48845) (width 0.2) (layer "F.Cu") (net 5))
 (segment (start 135.73125 123.03125) (end 136.36625 123.66625) (width 0.2) (layer "F.Cu") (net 5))
 (segment (start 135.73125 114.3) (end 135.73125 123.03125) (width 0.2) (layer "F.Cu") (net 5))
 (segment (start 169.87075 107.48845) (end 167.0197 110.3395) (width 0.2) (layer "F.Cu") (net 5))
 (segment (start 139.69175 110.3395) (end 135.73125 114.3) (width 0.2) (layer "F.Cu") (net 5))
 (segment (start 167.0197 110.3395) (end 139.69175 110.3395) (width 0.2) (layer "F.Cu") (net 5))
 (segment (start 168.23375 73.81875) (end 169.87075 75.45575) (width 0.2) (layer "F.Cu") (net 5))
 (segment (start 152.99375 66.19875) (end 148.51475 66.19875) (width 0.2) (layer "F.Cu") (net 8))
 (segment (start 148.51475 66.19875) (end 148.0385 66.675) (width 0.2) (layer "F.Cu") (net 8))
 (segment (start 148.0385 78.1885) (end 148.0385 66.675) (width 0.2) (layer "F.Cu") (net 8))
 (segment (start 155.41625 85.56625) (end 148.0385 78.1885) (width 0.2) (layer "F.Cu") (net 8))
 (segment (start 160.011066 104.61625) (end 155.41625 104.61625) (width 0.2) (layer "F.Cu") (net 10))
 (segment (start 164.531316 109.1365) (end 160.011066 104.61625) (width 0.2) (layer "F.Cu") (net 10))
 (segment (start 148.757 68.73875) (end 148.4395 69.05625) (width 0.2) (layer "F.Cu") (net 10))
 (segment (start 148.4395 69.05625) (end 148.4395 76.44315) (width 0.2) (layer "F.Cu") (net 10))
 (segment (start 168.66775 83.91085) (end 168.66775 106.99015) (width 0.2) (layer "F.Cu") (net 10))
 (segment (start 150.01875 78.0224) (end 162.7793 78.0224) (width 0.2) (layer "F.Cu") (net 10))
 (segment (start 162.7793 78.0224) (end 168.66775 83.91085) (width 0.2) (layer "F.Cu") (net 10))
 (segment (start 168.66775 106.99015) (end 166.5214 109.1365) (width 0.2) (layer "F.Cu") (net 10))
 (segment (start 148.4395 76.44315) (end 150.01875 78.0224) (width 0.2) (layer "F.Cu") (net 10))
 (segment (start 166.5214 109.1365) (end 164.531316 109.1365) (width 0.2) (layer "F.Cu") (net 10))
 (segment (start 152.99375 68.73875) (end 148.757 68.73875) (width 0.2) (layer "F.Cu") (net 10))
 (segment (start 172.42825 71.4375) (end 172.42825 126.47505) (width 0.2) (layer "F.Cu") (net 4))
 (segment (start 159.54375 133.35) (end 155.41625 129.2225) (width 0.2) (layer "F.Cu") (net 4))
 (segment (start 165.5533 133.35) (end 159.54375 133.35) (width 0.2) (layer "F.Cu") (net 4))
 (segment (start 172.42825 126.47505) (end 165.5533 133.35) (width 0.2) (layer "F.Cu") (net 4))
 (segment (start 168.23375 71.27875) (end 172.2695 71.27875) (width 0.2) (layer "F.Cu") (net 4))
 (segment (start 172.2695 71.27875) (end 172.42825 71.4375) (width 0.2) (layer "F.Cu") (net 4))
 (segment (start 155.41625 129.2225) (end 155.41625 123.66625) (width 0.2) (layer "F.Cu") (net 4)))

